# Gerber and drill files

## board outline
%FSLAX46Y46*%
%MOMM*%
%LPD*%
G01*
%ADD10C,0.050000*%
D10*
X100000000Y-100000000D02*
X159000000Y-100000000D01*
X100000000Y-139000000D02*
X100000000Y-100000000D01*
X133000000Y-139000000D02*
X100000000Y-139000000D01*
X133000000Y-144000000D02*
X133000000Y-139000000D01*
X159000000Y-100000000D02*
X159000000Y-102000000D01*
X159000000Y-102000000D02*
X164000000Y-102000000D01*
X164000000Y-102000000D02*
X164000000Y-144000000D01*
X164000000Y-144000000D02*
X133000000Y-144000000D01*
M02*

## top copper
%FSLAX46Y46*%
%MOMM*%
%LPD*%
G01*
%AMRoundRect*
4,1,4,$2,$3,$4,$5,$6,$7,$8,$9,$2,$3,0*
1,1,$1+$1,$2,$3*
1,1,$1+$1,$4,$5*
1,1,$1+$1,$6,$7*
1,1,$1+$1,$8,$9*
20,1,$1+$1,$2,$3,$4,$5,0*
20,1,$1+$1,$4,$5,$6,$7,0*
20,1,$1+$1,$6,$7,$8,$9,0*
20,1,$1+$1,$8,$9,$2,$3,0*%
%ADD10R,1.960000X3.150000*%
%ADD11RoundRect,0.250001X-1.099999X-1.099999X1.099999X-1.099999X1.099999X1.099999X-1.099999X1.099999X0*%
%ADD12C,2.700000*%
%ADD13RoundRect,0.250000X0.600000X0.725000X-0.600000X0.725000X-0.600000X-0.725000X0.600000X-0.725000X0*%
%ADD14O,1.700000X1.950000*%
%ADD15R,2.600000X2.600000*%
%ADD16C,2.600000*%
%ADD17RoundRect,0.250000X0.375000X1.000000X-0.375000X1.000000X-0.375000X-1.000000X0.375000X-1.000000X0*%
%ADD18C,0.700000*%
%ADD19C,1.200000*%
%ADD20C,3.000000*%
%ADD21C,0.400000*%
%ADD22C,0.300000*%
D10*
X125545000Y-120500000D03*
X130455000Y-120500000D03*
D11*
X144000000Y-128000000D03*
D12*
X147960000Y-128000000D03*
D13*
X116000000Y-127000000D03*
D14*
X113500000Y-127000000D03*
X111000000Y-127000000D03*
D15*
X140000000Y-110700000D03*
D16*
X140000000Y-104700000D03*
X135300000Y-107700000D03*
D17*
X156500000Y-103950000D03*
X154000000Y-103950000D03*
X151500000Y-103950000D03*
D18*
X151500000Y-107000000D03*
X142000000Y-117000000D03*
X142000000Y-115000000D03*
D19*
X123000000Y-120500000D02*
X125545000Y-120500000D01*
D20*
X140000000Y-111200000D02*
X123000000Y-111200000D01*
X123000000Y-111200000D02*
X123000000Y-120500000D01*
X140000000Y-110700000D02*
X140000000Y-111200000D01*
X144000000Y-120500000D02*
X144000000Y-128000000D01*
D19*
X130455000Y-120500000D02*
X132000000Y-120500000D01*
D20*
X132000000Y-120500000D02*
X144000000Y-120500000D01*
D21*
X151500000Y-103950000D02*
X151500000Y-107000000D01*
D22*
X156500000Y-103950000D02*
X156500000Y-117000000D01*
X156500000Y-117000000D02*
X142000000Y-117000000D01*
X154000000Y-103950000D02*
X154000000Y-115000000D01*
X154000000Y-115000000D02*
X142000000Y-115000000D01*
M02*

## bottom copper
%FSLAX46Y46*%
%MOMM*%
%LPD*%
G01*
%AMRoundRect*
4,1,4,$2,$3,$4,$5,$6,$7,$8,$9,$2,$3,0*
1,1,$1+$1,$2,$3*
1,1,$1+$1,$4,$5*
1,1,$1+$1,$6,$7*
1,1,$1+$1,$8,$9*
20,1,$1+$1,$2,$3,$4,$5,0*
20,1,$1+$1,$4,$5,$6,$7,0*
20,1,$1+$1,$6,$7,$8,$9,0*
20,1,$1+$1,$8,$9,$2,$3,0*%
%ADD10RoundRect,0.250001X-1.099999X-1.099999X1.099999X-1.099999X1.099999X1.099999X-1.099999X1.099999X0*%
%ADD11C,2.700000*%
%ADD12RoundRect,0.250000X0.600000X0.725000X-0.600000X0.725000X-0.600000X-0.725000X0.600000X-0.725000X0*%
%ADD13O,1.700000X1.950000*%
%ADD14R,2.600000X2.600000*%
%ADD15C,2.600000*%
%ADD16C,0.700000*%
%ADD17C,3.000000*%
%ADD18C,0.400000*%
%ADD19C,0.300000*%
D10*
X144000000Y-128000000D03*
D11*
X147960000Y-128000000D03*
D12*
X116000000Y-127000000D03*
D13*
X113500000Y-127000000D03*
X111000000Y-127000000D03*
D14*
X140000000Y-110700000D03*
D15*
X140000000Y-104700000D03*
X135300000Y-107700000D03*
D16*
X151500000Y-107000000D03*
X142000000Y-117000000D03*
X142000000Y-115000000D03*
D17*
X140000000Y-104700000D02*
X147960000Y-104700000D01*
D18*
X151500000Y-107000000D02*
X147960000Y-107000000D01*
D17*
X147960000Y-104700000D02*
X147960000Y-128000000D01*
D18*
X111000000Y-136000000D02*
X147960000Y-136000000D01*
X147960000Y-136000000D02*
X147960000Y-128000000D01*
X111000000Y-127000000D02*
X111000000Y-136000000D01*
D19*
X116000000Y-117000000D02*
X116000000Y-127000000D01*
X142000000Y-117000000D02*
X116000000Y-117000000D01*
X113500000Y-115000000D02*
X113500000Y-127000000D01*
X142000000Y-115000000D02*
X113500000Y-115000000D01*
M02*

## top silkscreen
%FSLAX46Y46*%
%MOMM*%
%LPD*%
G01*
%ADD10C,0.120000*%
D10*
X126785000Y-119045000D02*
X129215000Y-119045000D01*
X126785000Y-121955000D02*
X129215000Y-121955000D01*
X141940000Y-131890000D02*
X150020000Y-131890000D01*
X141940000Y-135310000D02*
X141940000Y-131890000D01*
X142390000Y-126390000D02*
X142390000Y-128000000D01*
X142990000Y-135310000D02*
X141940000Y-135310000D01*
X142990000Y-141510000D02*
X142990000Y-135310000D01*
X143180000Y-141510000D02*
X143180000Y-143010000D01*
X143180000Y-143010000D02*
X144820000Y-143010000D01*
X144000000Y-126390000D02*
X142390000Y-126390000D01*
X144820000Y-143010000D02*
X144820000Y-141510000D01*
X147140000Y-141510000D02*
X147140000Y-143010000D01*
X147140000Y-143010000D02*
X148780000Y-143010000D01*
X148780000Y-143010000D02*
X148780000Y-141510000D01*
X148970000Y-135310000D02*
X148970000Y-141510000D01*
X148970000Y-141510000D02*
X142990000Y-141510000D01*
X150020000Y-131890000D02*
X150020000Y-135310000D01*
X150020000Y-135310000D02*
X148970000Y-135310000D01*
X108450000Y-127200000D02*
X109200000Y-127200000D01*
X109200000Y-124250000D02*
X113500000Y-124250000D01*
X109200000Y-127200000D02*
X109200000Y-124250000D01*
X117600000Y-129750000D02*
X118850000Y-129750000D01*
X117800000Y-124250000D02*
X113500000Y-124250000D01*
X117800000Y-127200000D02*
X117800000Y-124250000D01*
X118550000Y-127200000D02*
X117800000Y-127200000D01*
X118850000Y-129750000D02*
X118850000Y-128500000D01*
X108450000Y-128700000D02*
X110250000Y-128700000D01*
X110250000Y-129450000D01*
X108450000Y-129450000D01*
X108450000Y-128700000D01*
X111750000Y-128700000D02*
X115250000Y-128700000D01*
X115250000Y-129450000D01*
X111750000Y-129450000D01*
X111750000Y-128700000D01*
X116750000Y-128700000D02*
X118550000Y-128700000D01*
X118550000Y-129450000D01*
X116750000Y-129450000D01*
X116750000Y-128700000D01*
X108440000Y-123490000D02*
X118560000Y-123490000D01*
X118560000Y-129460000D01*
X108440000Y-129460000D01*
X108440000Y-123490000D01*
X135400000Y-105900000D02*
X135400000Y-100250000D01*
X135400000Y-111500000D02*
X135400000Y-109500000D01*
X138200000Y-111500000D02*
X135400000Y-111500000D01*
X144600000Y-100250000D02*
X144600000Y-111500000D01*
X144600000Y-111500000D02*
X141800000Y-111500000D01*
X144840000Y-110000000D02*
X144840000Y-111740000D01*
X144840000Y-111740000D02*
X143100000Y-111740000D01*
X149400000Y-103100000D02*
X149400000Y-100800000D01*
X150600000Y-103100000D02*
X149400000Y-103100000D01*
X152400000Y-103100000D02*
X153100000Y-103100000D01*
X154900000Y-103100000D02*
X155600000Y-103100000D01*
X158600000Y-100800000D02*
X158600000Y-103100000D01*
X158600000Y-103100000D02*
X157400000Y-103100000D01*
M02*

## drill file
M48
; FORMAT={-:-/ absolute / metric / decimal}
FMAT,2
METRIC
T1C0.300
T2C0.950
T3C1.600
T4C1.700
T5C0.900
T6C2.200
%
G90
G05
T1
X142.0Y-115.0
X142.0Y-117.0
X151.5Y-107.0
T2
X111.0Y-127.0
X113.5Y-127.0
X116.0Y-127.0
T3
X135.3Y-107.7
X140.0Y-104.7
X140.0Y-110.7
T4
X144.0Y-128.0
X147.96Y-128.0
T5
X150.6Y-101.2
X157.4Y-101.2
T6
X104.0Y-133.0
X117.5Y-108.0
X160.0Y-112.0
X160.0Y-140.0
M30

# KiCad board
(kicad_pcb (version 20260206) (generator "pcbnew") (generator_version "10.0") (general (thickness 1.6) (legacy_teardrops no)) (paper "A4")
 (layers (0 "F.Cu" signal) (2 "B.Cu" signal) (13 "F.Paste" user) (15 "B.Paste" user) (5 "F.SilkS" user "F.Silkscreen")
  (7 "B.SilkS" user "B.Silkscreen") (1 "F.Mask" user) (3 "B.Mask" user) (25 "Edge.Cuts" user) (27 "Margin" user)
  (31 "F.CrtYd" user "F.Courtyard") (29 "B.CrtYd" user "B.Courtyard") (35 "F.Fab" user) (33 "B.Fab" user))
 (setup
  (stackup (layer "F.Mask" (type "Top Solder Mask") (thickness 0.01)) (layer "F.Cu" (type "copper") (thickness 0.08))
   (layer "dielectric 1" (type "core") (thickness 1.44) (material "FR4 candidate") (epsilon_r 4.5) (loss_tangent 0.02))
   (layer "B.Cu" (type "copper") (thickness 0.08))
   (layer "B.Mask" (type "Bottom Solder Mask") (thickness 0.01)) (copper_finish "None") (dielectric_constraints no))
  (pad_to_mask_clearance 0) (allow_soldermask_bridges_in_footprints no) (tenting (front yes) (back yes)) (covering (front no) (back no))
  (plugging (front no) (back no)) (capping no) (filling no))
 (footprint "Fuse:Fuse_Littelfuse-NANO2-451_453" (layer "F.Cu") (at 128 120.5)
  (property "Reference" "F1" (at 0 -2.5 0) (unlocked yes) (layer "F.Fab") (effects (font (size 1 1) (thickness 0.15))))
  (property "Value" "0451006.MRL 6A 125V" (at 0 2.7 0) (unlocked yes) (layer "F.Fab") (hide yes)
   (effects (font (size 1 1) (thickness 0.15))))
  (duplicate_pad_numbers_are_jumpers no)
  (fp_line (start -1.215 -1.455) (end 1.215 -1.455) (stroke (width 0.12) (type solid)) (layer "F.SilkS"))
  (fp_line (start -1.215 1.455) (end 1.215 1.455) (stroke (width 0.12) (type solid)) (layer "F.SilkS"))
  (pad "1" smd rect (at -2.455 0) (size 1.96 3.15) (layers "F.Cu" "F.Mask" "F.Paste") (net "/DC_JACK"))
  (pad "2" smd rect (at 2.455 0) (size 1.96 3.15) (layers "F.Cu" "F.Mask" "F.Paste") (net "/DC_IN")))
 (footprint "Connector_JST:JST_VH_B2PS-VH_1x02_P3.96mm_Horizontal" (layer "F.Cu") (at 144 128)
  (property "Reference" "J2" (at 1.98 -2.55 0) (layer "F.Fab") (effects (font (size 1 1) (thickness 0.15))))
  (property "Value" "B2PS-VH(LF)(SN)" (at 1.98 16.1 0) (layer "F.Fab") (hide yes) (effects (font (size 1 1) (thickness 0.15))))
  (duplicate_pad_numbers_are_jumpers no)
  (fp_line (start -2.06 3.89) (end 6.02 3.89) (stroke (width 0.12) (type solid)) (layer "F.SilkS"))
  (fp_line (start -2.06 7.31) (end -2.06 3.89) (stroke (width 0.12) (type solid)) (layer "F.SilkS"))
  (fp_line (start -1.61 -1.61) (end -1.61 0) (stroke (width 0.12) (type solid)) (layer "F.SilkS"))
  (fp_line (start -1.01 7.31) (end -2.06 7.31) (stroke (width 0.12) (type solid)) (layer "F.SilkS"))
  (fp_line (start -1.01 13.51) (end -1.01 7.31) (stroke (width 0.12) (type solid)) (layer "F.SilkS"))
  (fp_line (start -0.82 13.51) (end -0.82 15.01) (stroke (width 0.12) (type solid)) (layer "F.SilkS"))
  (fp_line (start -0.82 15.01) (end 0.82 15.01) (stroke (width 0.12) (type solid)) (layer "F.SilkS"))
  (fp_line (start 0 -1.61) (end -1.61 -1.61) (stroke (width 0.12) (type solid)) (layer "F.SilkS"))
  (fp_line (start 0.82 15.01) (end 0.82 13.51) (stroke (width 0.12) (type solid)) (layer "F.SilkS"))
  (fp_line (start 3.14 13.51) (end 3.14 15.01) (stroke (width 0.12) (type solid)) (layer "F.SilkS"))
  (fp_line (start 3.14 15.01) (end 4.78 15.01) (stroke (width 0.12) (type solid)) (layer "F.SilkS"))
  (fp_line (start 4.78 15.01) (end 4.78 13.51) (stroke (width 0.12) (type solid)) (layer "F.SilkS"))
  (fp_line (start 4.97 7.31) (end 4.97 13.51) (stroke (width 0.12) (type solid)) (layer "F.SilkS"))
  (fp_line (start 4.97 13.51) (end -1.01 13.51) (stroke (width 0.12) (type solid)) (layer "F.SilkS"))
  (fp_line (start 6.02 3.89) (end 6.02 7.31) (stroke (width 0.12) (type solid)) (layer "F.SilkS"))
  (fp_line (start 6.02 7.31) (end 4.97 7.31) (stroke (width 0.12) (type solid)) (layer "F.SilkS"))
  (pad "1" thru_hole roundrect (at 0 0) (size 2.7 2.7) (drill 1.7) (layers "*.Cu" "*.Mask") (remove_unused_layers no)
   (roundrect_rratio 0.092593) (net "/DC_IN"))
  (pad "2" thru_hole circle (at 3.96 0) (size 2.7 2.7) (drill 1.7) (layers "*.Cu" "*.Mask") (remove_unused_layers no) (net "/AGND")))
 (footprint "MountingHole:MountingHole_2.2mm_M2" (layer "F.Cu") (at 104 133)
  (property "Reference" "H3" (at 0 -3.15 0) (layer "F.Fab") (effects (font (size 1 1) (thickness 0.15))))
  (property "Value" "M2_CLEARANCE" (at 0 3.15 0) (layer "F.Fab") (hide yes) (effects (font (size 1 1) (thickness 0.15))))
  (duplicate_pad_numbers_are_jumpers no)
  (pad "" np_thru_hole circle (at 0 0) (size 2.2 2.2) (drill 2.2) (layers "*.Cu" "*.Mask")))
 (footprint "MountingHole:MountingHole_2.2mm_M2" (layer "F.Cu") (at 160 112)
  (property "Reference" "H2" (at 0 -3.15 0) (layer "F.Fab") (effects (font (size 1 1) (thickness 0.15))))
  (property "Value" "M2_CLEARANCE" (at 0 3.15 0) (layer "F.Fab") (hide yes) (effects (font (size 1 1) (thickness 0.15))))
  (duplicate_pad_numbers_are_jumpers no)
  (pad "" np_thru_hole circle (at 0 0) (size 2.2 2.2) (drill 2.2) (layers "*.Cu" "*.Mask")))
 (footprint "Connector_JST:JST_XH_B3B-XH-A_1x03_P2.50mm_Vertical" (layer "F.Cu") (at 116 127 180)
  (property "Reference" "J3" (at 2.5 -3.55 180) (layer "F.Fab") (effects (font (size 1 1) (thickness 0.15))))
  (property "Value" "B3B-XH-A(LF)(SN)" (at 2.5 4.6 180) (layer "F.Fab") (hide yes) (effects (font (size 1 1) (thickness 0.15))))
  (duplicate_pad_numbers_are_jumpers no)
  (fp_line (start 7.55 -0.2) (end 6.8 -0.2) (stroke (width 0.12) (type solid)) (layer "F.SilkS"))
  (fp_line (start 6.8 2.75) (end 2.5 2.75) (stroke (width 0.12) (type solid)) (layer "F.SilkS"))
  (fp_line (start 6.8 -0.2) (end 6.8 2.75) (stroke (width 0.12) (type solid)) (layer "F.SilkS"))
  (fp_line (start -1.6 -2.75) (end -2.85 -2.75) (stroke (width 0.12) (type solid)) (layer "F.SilkS"))
  (fp_line (start -1.8 2.75) (end 2.5 2.75) (stroke (width 0.12) (type solid)) (layer "F.SilkS"))
  (fp_line (start -1.8 -0.2) (end -1.8 2.75) (stroke (width 0.12) (type solid)) (layer "F.SilkS"))
  (fp_line (start -2.55 -0.2) (end -1.8 -0.2) (stroke (width 0.12) (type solid)) (layer "F.SilkS"))
  (fp_line (start -2.85 -2.75) (end -2.85 -1.5) (stroke (width 0.12) (type solid)) (layer "F.SilkS"))
  (fp_rect (start 5.75 -2.45) (end 7.55 -1.7) (stroke (width 0.12) (type solid)) (fill no) (layer "F.SilkS"))
  (fp_rect (start 0.75 -2.45) (end 4.25 -1.7) (stroke (width 0.12) (type solid)) (fill no) (layer "F.SilkS"))
  (fp_rect (start -2.55 -2.45) (end -0.75 -1.7) (stroke (width 0.12) (type solid)) (fill no) (layer "F.SilkS"))
  (fp_rect (start -2.56 -2.46) (end 7.56 3.51) (stroke (width 0.12) (type solid)) (fill no) (layer "F.SilkS"))
  (pad "1" thru_hole roundrect (at 0 0 180) (size 1.7 1.95) (drill 0.95) (layers "*.Cu" "*.Mask") (remove_unused_layers no)
   (roundrect_rratio 0.147059) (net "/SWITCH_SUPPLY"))
  (pad "2" thru_hole oval (at 2.5 0 180) (size 1.7 1.95) (drill 0.95) (layers "*.Cu" "*.Mask") (remove_unused_layers no) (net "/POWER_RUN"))
  (pad "3" thru_hole oval (at 5 0 180) (size 1.7 1.95) (drill 0.95) (layers "*.Cu" "*.Mask") (remove_unused_layers no) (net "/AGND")))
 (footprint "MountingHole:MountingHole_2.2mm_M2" (layer "F.Cu") (at 160 140)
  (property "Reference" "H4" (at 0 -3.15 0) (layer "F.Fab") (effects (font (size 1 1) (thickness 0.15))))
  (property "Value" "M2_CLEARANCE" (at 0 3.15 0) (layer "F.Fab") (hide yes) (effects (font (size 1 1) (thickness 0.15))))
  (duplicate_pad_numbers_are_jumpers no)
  (pad "" np_thru_hole circle (at 0 0) (size 2.2 2.2) (drill 2.2) (layers "*.Cu" "*.Mask")))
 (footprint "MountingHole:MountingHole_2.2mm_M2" (layer "F.Cu") (at 117.5 108)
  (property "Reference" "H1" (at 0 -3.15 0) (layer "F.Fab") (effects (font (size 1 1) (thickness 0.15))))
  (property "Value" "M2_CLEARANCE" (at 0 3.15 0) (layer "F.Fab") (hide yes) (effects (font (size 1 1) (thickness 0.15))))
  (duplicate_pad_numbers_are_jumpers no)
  (pad "" np_thru_hole circle (at 0 0) (size 2.2 2.2) (drill 2.2) (layers "*.Cu" "*.Mask")))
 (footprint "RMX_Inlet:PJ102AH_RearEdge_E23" (layer "F.Cu") (at 140 110.7 180)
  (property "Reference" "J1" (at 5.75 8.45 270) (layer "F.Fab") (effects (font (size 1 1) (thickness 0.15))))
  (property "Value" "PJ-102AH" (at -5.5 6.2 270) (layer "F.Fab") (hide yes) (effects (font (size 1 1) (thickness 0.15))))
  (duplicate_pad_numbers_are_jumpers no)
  (fp_line (start 4.6 4.8) (end 4.6 10.45) (stroke (width 0.12) (type solid)) (layer "F.SilkS"))
  (fp_line (start 4.6 -0.8) (end 4.6 1.2) (stroke (width 0.12) (type solid)) (layer "F.SilkS"))
  (fp_line (start 1.8 -0.8) (end 4.6 -0.8) (stroke (width 0.12) (type solid)) (layer "F.SilkS"))
  (fp_line (start -4.6 10.45) (end -4.6 -0.8) (stroke (width 0.12) (type solid)) (layer "F.SilkS"))
  (fp_line (start -4.6 -0.8) (end -1.8 -0.8) (stroke (width 0.12) (type solid)) (layer "F.SilkS"))
  (fp_line (start -4.84 0.7) (end -4.84 -1.04) (stroke (width 0.12) (type solid)) (layer "F.SilkS"))
  (fp_line (start -4.84 -1.04) (end -3.1 -1.04) (stroke (width 0.12) (type solid)) (layer "F.SilkS"))
  (pad "1" thru_hole rect (at 0 0 180) (size 2.6 2.6) (drill 1.6) (layers "*.Cu" "*.Mask") (remove_unused_layers no) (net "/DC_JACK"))
  (pad "2" thru_hole circle (at 0 6 180) (size 2.6 2.6) (drill 1.6) (layers "*.Cu" "*.Mask") (remove_unused_layers no) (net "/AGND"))
  (pad "3" thru_hole circle (at 4.7 3 180) (size 2.6 2.6) (drill 1.6) (layers "*.Cu" "*.Mask") (remove_unused_layers no)
   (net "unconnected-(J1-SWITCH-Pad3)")))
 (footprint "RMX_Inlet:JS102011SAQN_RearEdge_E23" (layer "F.Cu") (at 154 101.2 180)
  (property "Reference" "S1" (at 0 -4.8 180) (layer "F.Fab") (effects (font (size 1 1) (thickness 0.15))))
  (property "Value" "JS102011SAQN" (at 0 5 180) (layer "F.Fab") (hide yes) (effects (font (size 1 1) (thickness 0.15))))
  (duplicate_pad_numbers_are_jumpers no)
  (fp_line (start 4.6 -1.9) (end 4.6 0.4) (stroke (width 0.12) (type solid)) (layer "F.SilkS"))
  (fp_line (start 3.4 -1.9) (end 4.6 -1.9) (stroke (width 0.12) (type solid)) (layer "F.SilkS"))
  (fp_line (start 1.6 -1.9) (end 0.9 -1.9) (stroke (width 0.12) (type solid)) (layer "F.SilkS"))
  (fp_line (start -0.9 -1.9) (end -1.6 -1.9) (stroke (width 0.12) (type solid)) (layer "F.SilkS"))
  (fp_line (start -4.6 0.4) (end -4.6 -1.9) (stroke (width 0.12) (type solid)) (layer "F.SilkS"))
  (fp_line (start -4.6 -1.9) (end -3.4 -1.9) (stroke (width 0.12) (type solid)) (layer "F.SilkS"))
  (pad "" np_thru_hole circle (at -3.4 0 180) (size 0.9 0.9) (drill 0.9) (layers "*.Cu" "*.Mask"))
  (pad "" np_thru_hole circle (at 3.4 0 180) (size 0.9 0.9) (drill 0.9) (layers "*.Cu" "*.Mask"))
  (pad "1" smd roundrect (at -2.5 -2.75 180) (size 1.25 2.5) (layers "F.Cu" "F.Mask" "F.Paste") (roundrect_rratio 0.2)
   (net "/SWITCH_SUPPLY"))
  (pad "2" smd roundrect (at 0 -2.75 180) (size 1.25 2.5) (layers "F.Cu" "F.Mask" "F.Paste") (roundrect_rratio 0.2) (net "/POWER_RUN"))
  (pad "3" smd roundrect (at 2.5 -2.75 180) (size 1.25 2.5) (layers "F.Cu" "F.Mask" "F.Paste") (roundrect_rratio 0.2) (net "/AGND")))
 (gr_line (start 100 100) (end 159 100) (stroke (width 0.05) (type default)) (layer "Edge.Cuts"))
 (gr_line (start 100 139) (end 100 100) (stroke (width 0.05) (type default)) (layer "Edge.Cuts"))
 (gr_line (start 133 139) (end 100 139) (stroke (width 0.05) (type default)) (layer "Edge.Cuts"))
 (gr_line (start 133 144) (end 133 139) (stroke (width 0.05) (type default)) (layer "Edge.Cuts"))
 (gr_line (start 159 100) (end 159 102) (stroke (width 0.05) (type default)) (layer "Edge.Cuts"))
 (gr_line (start 159 102) (end 164 102) (stroke (width 0.05) (type default)) (layer "Edge.Cuts"))
 (gr_line (start 164 102) (end 164 144) (stroke (width 0.05) (type default)) (layer "Edge.Cuts"))
 (gr_line (start 164 144) (end 133 144) (stroke (width 0.05) (type default)) (layer "Edge.Cuts"))
 (segment (start 123 120.5) (end 125.545 120.5) (width 1.2) (layer "F.Cu") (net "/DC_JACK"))
 (segment (start 140 111.2) (end 123 111.2) (width 3) (layer "F.Cu") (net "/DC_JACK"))
 (segment (start 123 111.2) (end 123 120.5) (width 3) (layer "F.Cu") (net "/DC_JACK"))
 (segment (start 140 110.7) (end 140 111.2) (width 3) (layer "F.Cu") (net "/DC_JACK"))
 (segment (start 144 120.5) (end 144 128) (width 3) (layer "F.Cu") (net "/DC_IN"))
 (segment (start 130.455 120.5) (end 132 120.5) (width 1.2) (layer "F.Cu") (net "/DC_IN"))
 (segment (start 132 120.5) (end 144 120.5) (width 3) (layer "F.Cu") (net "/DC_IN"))
 (segment (start 151.5 103.95) (end 151.5 107) (width 0.4) (layer "F.Cu") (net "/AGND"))
 (via (at 151.5 107) (size 0.7) (drill 0.3) (layers "F.Cu" "B.Cu") (capping no) (covering (front no) (back no))
  (plugging (front no) (back no)) (filling no) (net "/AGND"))
 (segment (start 140 104.7) (end 147.96 104.7) (width 3) (layer "B.Cu") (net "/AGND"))
 (segment (start 151.5 107) (end 147.96 107) (width 0.4) (layer "B.Cu") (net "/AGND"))
 (segment (start 147.96 104.7) (end 147.96 128) (width 3) (layer "B.Cu") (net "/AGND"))
 (segment (start 111 136) (end 147.96 136) (width 0.4) (layer "B.Cu") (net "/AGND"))
 (segment (start 147.96 136) (end 147.96 128) (width 0.4) (layer "B.Cu") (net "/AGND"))
 (segment (start 111 127) (end 111 136) (width 0.4) (layer "B.Cu") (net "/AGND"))
 (segment (start 156.5 103.95) (end 156.5 117) (width 0.3) (layer "F.Cu") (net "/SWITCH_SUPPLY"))
 (segment (start 156.5 117) (end 142 117) (width 0.3) (layer "F.Cu") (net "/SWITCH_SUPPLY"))
 (via (at 142 117) (size 0.7) (drill 0.3) (layers "F.Cu" "B.Cu") (capping no) (covering (front no) (back no))
  (plugging (front no) (back no)) (filling no) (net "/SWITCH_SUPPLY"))
 (segment (start 116 117) (end 116 127) (width 0.3) (layer "B.Cu") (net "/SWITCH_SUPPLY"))
 (segment (start 142 117) (end 116 117) (width 0.3) (layer "B.Cu") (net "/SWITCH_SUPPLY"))
 (segment (start 154 103.95) (end 154 115) (width 0.3) (layer "F.Cu") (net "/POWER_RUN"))
 (segment (start 154 115) (end 142 115) (width 0.3) (layer "F.Cu") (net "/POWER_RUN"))
 (via (at 142 115) (size 0.7) (drill 0.3) (layers "F.Cu" "B.Cu") (capping no) (covering (front no) (back no))
  (plugging (front no) (back no)) (filling no) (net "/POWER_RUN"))
 (segment (start 113.5 115) (end 113.5 127) (width 0.3) (layer "B.Cu") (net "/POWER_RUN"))
 (segment (start 142 115) (end 113.5 115) (width 0.3) (layer "B.Cu") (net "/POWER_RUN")))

